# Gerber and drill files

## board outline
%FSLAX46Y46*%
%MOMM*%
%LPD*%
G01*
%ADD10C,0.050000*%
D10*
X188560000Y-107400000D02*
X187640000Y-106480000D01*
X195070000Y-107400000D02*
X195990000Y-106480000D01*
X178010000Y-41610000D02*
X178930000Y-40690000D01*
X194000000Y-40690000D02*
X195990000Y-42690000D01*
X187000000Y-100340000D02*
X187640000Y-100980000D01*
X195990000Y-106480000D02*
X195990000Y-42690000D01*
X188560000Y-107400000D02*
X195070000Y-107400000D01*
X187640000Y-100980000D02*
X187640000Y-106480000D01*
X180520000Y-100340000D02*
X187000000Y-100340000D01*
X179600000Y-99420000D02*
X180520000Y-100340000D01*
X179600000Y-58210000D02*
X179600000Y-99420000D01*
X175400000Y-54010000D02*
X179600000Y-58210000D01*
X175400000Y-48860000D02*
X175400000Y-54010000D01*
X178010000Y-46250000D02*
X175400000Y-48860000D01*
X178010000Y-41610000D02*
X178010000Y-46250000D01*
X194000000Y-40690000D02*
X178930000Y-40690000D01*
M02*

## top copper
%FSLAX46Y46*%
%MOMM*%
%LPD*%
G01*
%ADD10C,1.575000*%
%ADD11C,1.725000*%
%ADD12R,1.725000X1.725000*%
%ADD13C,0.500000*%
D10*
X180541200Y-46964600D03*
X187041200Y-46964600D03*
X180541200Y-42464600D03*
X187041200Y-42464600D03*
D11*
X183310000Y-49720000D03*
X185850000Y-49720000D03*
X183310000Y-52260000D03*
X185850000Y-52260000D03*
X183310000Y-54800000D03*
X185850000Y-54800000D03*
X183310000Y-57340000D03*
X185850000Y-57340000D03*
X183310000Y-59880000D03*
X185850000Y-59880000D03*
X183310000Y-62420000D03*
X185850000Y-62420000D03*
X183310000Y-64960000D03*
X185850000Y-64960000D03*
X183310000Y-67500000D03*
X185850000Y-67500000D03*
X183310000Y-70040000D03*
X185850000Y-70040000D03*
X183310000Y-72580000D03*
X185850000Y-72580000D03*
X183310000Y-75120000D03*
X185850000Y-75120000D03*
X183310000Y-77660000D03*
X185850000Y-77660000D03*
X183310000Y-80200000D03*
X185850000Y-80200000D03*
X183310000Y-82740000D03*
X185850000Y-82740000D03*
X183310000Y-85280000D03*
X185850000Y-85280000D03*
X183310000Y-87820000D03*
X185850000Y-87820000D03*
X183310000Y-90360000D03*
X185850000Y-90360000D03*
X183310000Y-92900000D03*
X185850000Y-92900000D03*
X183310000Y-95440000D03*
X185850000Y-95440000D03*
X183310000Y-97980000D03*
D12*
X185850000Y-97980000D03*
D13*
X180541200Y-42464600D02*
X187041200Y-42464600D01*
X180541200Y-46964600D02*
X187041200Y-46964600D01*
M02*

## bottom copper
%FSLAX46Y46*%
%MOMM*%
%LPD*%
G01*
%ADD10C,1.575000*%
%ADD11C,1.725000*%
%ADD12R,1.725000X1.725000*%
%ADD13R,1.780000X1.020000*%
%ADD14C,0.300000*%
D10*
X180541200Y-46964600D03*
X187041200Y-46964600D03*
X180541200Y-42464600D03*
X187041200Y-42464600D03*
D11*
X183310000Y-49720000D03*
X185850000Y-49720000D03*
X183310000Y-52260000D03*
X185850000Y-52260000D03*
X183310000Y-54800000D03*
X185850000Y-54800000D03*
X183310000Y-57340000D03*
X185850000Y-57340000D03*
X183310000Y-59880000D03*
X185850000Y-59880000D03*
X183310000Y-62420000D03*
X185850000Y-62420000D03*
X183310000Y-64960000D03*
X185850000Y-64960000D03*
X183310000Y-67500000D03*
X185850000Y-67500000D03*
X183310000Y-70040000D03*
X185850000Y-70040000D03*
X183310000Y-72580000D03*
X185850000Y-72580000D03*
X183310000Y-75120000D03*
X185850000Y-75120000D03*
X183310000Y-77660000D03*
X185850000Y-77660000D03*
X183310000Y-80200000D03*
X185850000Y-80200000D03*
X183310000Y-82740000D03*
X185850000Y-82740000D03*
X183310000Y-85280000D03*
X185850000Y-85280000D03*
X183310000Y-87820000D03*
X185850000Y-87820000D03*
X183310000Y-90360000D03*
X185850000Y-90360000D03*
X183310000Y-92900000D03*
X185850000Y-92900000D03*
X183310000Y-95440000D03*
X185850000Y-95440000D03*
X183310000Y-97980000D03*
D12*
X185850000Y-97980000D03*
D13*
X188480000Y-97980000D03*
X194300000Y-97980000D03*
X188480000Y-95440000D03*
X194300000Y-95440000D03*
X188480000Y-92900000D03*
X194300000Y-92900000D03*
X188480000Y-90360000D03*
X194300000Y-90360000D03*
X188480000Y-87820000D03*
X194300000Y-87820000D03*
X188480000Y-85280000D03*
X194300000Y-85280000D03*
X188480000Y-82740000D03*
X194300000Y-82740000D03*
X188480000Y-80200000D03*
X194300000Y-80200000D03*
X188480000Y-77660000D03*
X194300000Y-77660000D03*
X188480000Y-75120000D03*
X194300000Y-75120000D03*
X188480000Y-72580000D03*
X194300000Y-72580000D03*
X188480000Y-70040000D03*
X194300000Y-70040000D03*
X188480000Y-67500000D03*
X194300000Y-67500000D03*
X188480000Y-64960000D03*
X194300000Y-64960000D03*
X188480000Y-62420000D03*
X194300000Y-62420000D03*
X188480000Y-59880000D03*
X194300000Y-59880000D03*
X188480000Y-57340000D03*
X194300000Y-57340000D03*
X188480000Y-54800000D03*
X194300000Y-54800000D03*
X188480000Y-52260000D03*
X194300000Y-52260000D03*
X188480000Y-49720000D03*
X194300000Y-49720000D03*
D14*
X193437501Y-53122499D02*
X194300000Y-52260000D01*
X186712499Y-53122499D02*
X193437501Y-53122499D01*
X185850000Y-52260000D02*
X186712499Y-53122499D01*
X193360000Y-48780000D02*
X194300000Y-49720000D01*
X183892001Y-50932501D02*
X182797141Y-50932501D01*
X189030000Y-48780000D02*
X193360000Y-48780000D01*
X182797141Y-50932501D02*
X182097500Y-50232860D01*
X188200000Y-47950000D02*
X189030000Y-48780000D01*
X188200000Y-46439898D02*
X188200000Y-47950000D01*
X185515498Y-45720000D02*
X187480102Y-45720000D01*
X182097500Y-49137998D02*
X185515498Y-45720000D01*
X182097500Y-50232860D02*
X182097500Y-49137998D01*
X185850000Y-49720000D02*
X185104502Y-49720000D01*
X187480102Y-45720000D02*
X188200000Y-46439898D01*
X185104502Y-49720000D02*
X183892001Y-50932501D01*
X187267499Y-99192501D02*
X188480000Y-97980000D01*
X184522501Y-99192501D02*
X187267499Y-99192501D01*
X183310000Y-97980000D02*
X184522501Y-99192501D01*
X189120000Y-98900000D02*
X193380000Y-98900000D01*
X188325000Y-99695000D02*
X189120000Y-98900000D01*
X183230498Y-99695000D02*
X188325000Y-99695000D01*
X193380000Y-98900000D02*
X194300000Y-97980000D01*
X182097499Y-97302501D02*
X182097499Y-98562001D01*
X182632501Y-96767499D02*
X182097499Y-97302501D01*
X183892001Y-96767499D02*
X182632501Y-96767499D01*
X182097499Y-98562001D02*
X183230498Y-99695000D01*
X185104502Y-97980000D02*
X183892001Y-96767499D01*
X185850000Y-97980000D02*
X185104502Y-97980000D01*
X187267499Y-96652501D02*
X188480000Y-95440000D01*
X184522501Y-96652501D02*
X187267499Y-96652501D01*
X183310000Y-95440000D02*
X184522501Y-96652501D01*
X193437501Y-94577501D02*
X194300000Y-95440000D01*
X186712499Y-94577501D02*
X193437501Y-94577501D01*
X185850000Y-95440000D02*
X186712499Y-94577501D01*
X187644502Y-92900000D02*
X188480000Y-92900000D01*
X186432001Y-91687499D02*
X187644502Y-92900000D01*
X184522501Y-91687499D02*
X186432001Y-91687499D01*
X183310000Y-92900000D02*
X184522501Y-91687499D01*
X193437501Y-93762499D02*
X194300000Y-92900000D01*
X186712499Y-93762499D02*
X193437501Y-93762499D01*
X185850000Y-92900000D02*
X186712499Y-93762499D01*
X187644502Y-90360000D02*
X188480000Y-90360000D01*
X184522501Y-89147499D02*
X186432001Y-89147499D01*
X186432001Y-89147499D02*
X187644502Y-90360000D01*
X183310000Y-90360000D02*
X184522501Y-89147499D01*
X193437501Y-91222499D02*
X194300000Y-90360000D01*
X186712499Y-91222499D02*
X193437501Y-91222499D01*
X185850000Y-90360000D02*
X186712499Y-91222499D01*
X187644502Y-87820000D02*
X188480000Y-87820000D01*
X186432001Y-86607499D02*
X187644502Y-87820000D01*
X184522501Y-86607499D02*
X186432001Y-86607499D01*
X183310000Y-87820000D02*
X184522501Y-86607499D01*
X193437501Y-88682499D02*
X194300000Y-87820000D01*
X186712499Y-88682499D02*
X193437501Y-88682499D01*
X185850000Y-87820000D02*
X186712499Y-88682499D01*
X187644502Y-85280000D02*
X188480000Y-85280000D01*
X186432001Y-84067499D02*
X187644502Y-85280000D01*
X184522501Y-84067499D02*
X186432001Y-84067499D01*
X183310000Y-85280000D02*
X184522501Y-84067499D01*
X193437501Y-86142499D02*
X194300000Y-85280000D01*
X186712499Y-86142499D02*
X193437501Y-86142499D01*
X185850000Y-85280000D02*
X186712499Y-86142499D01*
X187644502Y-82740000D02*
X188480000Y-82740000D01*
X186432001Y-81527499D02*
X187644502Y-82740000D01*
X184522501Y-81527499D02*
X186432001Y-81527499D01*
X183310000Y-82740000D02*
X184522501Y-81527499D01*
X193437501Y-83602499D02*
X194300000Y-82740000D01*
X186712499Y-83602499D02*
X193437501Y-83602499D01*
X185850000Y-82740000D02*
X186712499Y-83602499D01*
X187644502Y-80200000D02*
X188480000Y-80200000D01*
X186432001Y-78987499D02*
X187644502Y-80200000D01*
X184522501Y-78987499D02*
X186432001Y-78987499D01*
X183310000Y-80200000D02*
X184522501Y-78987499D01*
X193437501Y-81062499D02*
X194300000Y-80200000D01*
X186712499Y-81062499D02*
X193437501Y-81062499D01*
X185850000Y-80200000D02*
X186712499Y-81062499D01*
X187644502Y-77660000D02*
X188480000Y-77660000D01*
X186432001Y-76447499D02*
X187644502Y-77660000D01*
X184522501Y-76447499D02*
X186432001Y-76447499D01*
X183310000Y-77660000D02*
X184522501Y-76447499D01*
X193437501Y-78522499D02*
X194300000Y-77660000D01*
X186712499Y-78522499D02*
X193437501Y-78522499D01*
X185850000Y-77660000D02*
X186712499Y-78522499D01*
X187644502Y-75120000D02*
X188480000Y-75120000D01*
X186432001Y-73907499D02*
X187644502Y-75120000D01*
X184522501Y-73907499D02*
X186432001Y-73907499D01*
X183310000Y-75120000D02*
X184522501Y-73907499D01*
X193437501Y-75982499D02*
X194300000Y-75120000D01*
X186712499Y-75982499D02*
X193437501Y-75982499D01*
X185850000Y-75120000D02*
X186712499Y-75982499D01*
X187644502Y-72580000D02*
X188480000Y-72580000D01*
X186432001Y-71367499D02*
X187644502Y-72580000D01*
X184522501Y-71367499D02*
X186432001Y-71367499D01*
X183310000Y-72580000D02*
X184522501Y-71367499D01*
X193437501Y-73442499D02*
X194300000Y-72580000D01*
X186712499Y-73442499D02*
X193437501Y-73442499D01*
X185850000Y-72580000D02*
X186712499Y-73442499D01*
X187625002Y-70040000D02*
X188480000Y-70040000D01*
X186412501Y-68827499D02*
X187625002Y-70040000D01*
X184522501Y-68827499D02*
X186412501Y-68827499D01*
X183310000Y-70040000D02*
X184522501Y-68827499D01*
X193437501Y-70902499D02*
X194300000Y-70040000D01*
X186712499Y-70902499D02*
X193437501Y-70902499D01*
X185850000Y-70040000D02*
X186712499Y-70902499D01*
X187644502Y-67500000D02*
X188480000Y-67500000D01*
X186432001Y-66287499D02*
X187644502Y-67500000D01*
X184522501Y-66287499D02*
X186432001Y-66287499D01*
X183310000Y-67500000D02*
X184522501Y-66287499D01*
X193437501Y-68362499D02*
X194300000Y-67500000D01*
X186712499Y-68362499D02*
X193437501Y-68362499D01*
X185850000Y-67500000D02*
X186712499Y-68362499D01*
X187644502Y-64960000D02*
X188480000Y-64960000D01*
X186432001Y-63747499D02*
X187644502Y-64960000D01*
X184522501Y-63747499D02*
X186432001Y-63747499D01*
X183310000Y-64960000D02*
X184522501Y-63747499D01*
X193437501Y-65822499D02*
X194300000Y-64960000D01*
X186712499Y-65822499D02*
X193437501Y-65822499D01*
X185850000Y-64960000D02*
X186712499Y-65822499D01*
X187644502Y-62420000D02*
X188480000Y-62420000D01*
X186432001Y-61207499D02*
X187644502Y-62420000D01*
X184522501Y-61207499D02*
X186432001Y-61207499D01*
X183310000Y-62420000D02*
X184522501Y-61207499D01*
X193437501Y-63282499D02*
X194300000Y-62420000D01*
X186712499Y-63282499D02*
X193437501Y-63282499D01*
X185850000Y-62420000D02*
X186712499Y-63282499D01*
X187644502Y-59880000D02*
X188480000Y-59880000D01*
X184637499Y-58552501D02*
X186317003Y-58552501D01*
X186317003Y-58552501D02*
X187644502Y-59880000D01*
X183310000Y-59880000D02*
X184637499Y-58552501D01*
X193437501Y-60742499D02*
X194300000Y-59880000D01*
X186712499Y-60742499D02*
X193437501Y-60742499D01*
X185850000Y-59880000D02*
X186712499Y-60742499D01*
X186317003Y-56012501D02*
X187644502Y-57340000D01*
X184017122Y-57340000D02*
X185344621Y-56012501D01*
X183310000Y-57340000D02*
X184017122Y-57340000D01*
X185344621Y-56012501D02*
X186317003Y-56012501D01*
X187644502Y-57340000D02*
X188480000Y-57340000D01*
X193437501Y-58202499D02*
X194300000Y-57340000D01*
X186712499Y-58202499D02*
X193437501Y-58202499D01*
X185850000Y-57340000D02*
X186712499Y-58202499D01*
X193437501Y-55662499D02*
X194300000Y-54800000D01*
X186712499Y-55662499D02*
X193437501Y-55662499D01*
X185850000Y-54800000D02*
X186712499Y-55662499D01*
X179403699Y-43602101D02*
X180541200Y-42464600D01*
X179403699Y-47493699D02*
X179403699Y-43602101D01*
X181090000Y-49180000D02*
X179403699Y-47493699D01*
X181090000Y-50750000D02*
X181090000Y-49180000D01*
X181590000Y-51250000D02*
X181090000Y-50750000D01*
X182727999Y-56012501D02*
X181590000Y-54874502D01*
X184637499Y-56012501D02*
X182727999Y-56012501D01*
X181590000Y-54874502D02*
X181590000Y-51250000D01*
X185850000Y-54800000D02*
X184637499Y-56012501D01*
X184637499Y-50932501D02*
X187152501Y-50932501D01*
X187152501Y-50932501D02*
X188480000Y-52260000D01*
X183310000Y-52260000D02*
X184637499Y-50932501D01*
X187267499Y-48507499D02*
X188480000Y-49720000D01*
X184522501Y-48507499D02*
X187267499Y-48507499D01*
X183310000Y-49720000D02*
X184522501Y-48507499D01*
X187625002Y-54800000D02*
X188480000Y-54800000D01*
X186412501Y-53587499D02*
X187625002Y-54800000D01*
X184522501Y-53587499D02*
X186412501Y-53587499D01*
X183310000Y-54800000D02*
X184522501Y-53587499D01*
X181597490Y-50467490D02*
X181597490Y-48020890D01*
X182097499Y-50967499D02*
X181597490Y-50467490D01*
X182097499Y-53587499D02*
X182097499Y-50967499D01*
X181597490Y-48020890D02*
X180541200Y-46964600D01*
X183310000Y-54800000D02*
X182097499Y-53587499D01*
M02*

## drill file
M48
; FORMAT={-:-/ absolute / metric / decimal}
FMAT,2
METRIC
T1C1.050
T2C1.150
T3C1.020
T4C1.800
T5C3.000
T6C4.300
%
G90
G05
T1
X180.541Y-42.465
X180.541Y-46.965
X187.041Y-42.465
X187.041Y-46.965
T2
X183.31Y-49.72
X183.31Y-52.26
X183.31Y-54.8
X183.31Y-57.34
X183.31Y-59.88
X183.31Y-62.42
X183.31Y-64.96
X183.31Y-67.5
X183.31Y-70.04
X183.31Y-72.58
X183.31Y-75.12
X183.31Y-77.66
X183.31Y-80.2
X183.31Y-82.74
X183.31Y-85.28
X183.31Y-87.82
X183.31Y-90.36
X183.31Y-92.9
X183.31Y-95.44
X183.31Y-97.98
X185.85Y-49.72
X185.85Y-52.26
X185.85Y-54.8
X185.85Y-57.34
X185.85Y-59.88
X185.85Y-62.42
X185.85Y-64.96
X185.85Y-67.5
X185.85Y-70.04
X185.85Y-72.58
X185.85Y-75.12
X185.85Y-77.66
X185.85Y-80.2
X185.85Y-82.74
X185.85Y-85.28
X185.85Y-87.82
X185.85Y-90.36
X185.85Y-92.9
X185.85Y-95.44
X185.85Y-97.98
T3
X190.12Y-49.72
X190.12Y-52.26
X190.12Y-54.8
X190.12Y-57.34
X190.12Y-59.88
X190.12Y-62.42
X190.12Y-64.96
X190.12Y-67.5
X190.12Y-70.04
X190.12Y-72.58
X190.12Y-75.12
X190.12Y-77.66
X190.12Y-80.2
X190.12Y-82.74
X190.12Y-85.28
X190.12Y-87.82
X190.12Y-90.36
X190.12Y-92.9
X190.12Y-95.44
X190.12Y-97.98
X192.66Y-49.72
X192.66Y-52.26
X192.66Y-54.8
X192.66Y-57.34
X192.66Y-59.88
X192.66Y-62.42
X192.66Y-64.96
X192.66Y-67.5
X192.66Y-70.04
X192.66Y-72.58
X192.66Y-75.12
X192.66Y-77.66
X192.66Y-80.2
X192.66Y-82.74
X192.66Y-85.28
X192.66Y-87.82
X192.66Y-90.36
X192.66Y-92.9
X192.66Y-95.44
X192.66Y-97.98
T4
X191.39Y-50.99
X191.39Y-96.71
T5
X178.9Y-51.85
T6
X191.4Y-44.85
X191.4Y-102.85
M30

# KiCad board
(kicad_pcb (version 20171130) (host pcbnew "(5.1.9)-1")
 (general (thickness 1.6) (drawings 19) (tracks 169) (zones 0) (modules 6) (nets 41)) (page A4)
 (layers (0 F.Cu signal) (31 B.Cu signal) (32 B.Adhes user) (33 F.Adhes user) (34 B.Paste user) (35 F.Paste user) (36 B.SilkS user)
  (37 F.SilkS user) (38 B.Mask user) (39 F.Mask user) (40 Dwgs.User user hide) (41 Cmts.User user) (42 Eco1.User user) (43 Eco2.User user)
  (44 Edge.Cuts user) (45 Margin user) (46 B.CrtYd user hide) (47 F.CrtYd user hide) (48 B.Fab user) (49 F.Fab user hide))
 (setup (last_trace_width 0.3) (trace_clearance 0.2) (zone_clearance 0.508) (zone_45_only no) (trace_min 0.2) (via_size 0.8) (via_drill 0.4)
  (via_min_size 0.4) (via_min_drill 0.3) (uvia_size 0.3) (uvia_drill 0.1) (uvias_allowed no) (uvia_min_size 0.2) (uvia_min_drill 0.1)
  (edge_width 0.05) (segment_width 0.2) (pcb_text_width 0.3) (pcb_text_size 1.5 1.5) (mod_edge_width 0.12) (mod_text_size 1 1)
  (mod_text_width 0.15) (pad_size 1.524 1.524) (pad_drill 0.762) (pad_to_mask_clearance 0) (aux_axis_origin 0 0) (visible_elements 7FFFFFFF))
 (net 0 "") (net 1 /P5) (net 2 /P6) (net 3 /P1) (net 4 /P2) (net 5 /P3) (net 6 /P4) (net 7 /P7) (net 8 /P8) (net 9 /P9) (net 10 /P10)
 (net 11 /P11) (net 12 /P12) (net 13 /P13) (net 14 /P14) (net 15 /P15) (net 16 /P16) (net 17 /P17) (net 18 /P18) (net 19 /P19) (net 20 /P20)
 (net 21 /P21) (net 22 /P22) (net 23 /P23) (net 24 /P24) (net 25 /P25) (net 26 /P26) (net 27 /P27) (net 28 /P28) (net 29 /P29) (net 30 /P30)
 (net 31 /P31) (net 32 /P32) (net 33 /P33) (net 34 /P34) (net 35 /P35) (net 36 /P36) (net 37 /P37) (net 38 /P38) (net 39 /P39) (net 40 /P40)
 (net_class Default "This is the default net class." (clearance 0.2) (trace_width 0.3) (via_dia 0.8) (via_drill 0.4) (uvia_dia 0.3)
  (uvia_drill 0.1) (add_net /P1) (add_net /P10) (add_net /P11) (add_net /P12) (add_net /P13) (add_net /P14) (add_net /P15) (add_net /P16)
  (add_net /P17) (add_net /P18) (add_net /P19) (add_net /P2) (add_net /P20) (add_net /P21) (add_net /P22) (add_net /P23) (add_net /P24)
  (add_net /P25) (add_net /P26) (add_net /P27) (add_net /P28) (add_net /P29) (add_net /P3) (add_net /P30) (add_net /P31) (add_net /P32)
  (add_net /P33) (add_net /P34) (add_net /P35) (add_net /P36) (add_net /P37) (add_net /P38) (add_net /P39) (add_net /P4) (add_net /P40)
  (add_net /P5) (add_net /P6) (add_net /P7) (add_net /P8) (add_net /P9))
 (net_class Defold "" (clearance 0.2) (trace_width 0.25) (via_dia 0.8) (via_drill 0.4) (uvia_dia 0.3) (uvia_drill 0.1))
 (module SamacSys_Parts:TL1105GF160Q (layer F.Cu) (at 183.7912 44.7146)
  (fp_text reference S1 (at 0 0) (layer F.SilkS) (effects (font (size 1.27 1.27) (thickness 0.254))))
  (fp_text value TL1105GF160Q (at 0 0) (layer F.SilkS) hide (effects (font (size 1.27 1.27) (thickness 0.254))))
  (pad 1 thru_hole circle (at -3.25 2.25) (size 1.575 1.575) (drill 1.05) (layers *.Cu *.Mask) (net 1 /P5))
  (pad 2 thru_hole circle (at 3.25 2.25) (size 1.575 1.575) (drill 1.05) (layers *.Cu *.Mask) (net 1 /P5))
  (pad 3 thru_hole circle (at -3.25 -2.25) (size 1.575 1.575) (drill 1.05) (layers *.Cu *.Mask) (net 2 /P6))
  (pad 4 thru_hole circle (at 3.25 -2.25) (size 1.575 1.575) (drill 1.05) (layers *.Cu *.Mask) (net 2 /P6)))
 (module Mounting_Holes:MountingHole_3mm (layer F.Cu) (at 178.9 51.85)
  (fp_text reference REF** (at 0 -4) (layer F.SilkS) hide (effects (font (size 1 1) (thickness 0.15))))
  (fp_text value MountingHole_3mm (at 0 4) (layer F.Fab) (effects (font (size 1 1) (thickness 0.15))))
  (pad 1 np_thru_hole circle (at 0 0) (size 3 3) (drill 3) (layers *.Cu *.Mask)))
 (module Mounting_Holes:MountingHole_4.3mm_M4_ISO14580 (layer F.Cu) (at 191.4 102.85)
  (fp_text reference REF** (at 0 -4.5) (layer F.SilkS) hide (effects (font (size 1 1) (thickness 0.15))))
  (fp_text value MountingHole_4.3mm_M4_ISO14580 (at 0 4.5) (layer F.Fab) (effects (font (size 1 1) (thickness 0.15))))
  (pad 1 np_thru_hole circle (at 0 0) (size 4.3 4.3) (drill 4.3) (layers *.Cu *.Mask)))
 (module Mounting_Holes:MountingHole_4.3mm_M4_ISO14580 (layer F.Cu) (at 191.4 44.85)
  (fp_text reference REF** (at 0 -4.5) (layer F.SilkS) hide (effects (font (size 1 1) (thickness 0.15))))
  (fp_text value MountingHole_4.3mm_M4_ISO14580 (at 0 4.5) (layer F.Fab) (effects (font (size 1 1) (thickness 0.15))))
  (pad 1 np_thru_hole circle (at 0 0) (size 4.3 4.3) (drill 4.3) (layers *.Cu *.Mask)))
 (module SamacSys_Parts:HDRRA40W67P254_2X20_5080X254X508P (layer F.Cu) (at 185.85 97.98 270)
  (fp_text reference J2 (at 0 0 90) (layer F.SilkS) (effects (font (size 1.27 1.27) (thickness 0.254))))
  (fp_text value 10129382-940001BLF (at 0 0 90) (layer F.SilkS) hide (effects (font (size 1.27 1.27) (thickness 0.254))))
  (pad 40 thru_hole circle (at -48.26 2.54 270) (size 1.725 1.725) (drill 1.15) (layers *.Cu *.Mask) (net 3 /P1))
  (pad 39 thru_hole circle (at -48.26 0 270) (size 1.725 1.725) (drill 1.15) (layers *.Cu *.Mask) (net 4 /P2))
  (pad 38 thru_hole circle (at -45.72 2.54 270) (size 1.725 1.725) (drill 1.15) (layers *.Cu *.Mask) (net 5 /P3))
  (pad 37 thru_hole circle (at -45.72 0 270) (size 1.725 1.725) (drill 1.15) (layers *.Cu *.Mask) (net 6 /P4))
  (pad 36 thru_hole circle (at -43.18 2.54 270) (size 1.725 1.725) (drill 1.15) (layers *.Cu *.Mask) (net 1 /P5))
  (pad 35 thru_hole circle (at -43.18 0 270) (size 1.725 1.725) (drill 1.15) (layers *.Cu *.Mask) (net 2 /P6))
  (pad 34 thru_hole circle (at -40.64 2.54 270) (size 1.725 1.725) (drill 1.15) (layers *.Cu *.Mask) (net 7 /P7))
  (pad 33 thru_hole circle (at -40.64 0 270) (size 1.725 1.725) (drill 1.15) (layers *.Cu *.Mask) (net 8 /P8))
  (pad 32 thru_hole circle (at -38.1 2.54 270) (size 1.725 1.725) (drill 1.15) (layers *.Cu *.Mask) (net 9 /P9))
  (pad 31 thru_hole circle (at -38.1 0 270) (size 1.725 1.725) (drill 1.15) (layers *.Cu *.Mask) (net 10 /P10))
  (pad 30 thru_hole circle (at -35.56 2.54 270) (size 1.725 1.725) (drill 1.15) (layers *.Cu *.Mask) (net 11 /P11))
  (pad 29 thru_hole circle (at -35.56 0 270) (size 1.725 1.725) (drill 1.15) (layers *.Cu *.Mask) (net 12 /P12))
  (pad 28 thru_hole circle (at -33.02 2.54 270) (size 1.725 1.725) (drill 1.15) (layers *.Cu *.Mask) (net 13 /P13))
  (pad 27 thru_hole circle (at -33.02 0 270) (size 1.725 1.725) (drill 1.15) (layers *.Cu *.Mask) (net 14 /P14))
  (pad 26 thru_hole circle (at -30.48 2.54 270) (size 1.725 1.725) (drill 1.15) (layers *.Cu *.Mask) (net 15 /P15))
  (pad 25 thru_hole circle (at -30.48 0 270) (size 1.725 1.725) (drill 1.15) (layers *.Cu *.Mask) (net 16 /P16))
  (pad 24 thru_hole circle (at -27.94 2.54 270) (size 1.725 1.725) (drill 1.15) (layers *.Cu *.Mask) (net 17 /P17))
  (pad 23 thru_hole circle (at -27.94 0 270) (size 1.725 1.725) (drill 1.15) (layers *.Cu *.Mask) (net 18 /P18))
  (pad 22 thru_hole circle (at -25.4 2.54 270) (size 1.725 1.725) (drill 1.15) (layers *.Cu *.Mask) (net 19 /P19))
  (pad 21 thru_hole circle (at -25.4 0 270) (size 1.725 1.725) (drill 1.15) (layers *.Cu *.Mask) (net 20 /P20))
  (pad 20 thru_hole circle (at -22.86 2.54 270) (size 1.725 1.725) (drill 1.15) (layers *.Cu *.Mask) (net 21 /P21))
  (pad 19 thru_hole circle (at -22.86 0 270) (size 1.725 1.725) (drill 1.15) (layers *.Cu *.Mask) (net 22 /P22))
  (pad 18 thru_hole circle (at -20.32 2.54 270) (size 1.725 1.725) (drill 1.15) (layers *.Cu *.Mask) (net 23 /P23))
  (pad 17 thru_hole circle (at -20.32 0 270) (size 1.725 1.725) (drill 1.15) (layers *.Cu *.Mask) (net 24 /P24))
  (pad 16 thru_hole circle (at -17.78 2.54 270) (size 1.725 1.725) (drill 1.15) (layers *.Cu *.Mask) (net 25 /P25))
  (pad 15 thru_hole circle (at -17.78 0 270) (size 1.725 1.725) (drill 1.15) (layers *.Cu *.Mask) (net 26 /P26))
  (pad 14 thru_hole circle (at -15.24 2.54 270) (size 1.725 1.725) (drill 1.15) (layers *.Cu *.Mask) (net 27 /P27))
  (pad 13 thru_hole circle (at -15.24 0 270) (size 1.725 1.725) (drill 1.15) (layers *.Cu *.Mask) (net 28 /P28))
  (pad 12 thru_hole circle (at -12.7 2.54 270) (size 1.725 1.725) (drill 1.15) (layers *.Cu *.Mask) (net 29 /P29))
  (pad 11 thru_hole circle (at -12.7 0 270) (size 1.725 1.725) (drill 1.15) (layers *.Cu *.Mask) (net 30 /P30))
  (pad 10 thru_hole circle (at -10.16 2.54 270) (size 1.725 1.725) (drill 1.15) (layers *.Cu *.Mask) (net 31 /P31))
  (pad 9 thru_hole circle (at -10.16 0 270) (size 1.725 1.725) (drill 1.15) (layers *.Cu *.Mask) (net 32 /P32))
  (pad 8 thru_hole circle (at -7.62 2.54 270) (size 1.725 1.725) (drill 1.15) (layers *.Cu *.Mask) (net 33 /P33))
  (pad 7 thru_hole circle (at -7.62 0 270) (size 1.725 1.725) (drill 1.15) (layers *.Cu *.Mask) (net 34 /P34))
  (pad 6 thru_hole circle (at -5.08 2.54 270) (size 1.725 1.725) (drill 1.15) (layers *.Cu *.Mask) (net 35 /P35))
  (pad 5 thru_hole circle (at -5.08 0 270) (size 1.725 1.725) (drill 1.15) (layers *.Cu *.Mask) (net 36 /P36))
  (pad 4 thru_hole circle (at -2.54 2.54 270) (size 1.725 1.725) (drill 1.15) (layers *.Cu *.Mask) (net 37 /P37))
  (pad 3 thru_hole circle (at -2.54 0 270) (size 1.725 1.725) (drill 1.15) (layers *.Cu *.Mask) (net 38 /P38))
  (pad 2 thru_hole circle (at 0 2.54 270) (size 1.725 1.725) (drill 1.15) (layers *.Cu *.Mask) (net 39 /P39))
  (pad 1 thru_hole rect (at 0 0 270) (size 1.725 1.725) (drill 1.15) (layers *.Cu *.Mask) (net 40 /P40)))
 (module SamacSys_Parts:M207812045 (layer B.Cu) (at 191.39 73.85 270)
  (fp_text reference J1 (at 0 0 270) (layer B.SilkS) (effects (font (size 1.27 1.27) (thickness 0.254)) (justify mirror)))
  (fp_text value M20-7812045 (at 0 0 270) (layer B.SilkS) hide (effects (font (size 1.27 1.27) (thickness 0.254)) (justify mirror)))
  (pad MH2 np_thru_hole circle (at 22.86 0 270) (size 1.8 0) (drill 1.8) (layers *.Cu *.Mask))
  (pad MH1 np_thru_hole circle (at -22.86 0 270) (size 1.8 0) (drill 1.8) (layers *.Cu *.Mask))
  (pad 80 np_thru_hole circle (at 24.13 1.27 270) (size 1.02 0) (drill 1.02) (layers *.Cu *.Mask))
  (pad 79 np_thru_hole circle (at 24.13 -1.27 270) (size 1.02 0) (drill 1.02) (layers *.Cu *.Mask))
  (pad 78 np_thru_hole circle (at 21.59 1.27 270) (size 1.02 0) (drill 1.02) (layers *.Cu *.Mask))
  (pad 77 np_thru_hole circle (at 21.59 -1.27 270) (size 1.02 0) (drill 1.02) (layers *.Cu *.Mask))
  (pad 76 np_thru_hole circle (at 19.05 1.27 270) (size 1.02 0) (drill 1.02) (layers *.Cu *.Mask))
  (pad 75 np_thru_hole circle (at 19.05 -1.27 270) (size 1.02 0) (drill 1.02) (layers *.Cu *.Mask))
  (pad 74 np_thru_hole circle (at 16.51 1.27 270) (size 1.02 0) (drill 1.02) (layers *.Cu *.Mask))
  (pad 73 np_thru_hole circle (at 16.51 -1.27 270) (size 1.02 0) (drill 1.02) (layers *.Cu *.Mask))
  (pad 72 np_thru_hole circle (at 13.97 1.27 270) (size 1.02 0) (drill 1.02) (layers *.Cu *.Mask))
  (pad 71 np_thru_hole circle (at 13.97 -1.27 270) (size 1.02 0) (drill 1.02) (layers *.Cu *.Mask))
  (pad 70 np_thru_hole circle (at 11.43 1.27 270) (size 1.02 0) (drill 1.02) (layers *.Cu *.Mask))
  (pad 69 np_thru_hole circle (at 11.43 -1.27 270) (size 1.02 0) (drill 1.02) (layers *.Cu *.Mask))
  (pad 68 np_thru_hole circle (at 8.89 1.27 270) (size 1.02 0) (drill 1.02) (layers *.Cu *.Mask))
  (pad 67 np_thru_hole circle (at 8.89 -1.27 270) (size 1.02 0) (drill 1.02) (layers *.Cu *.Mask))
  (pad 66 np_thru_hole circle (at 6.35 1.27 270) (size 1.02 0) (drill 1.02) (layers *.Cu *.Mask))
  (pad 65 np_thru_hole circle (at 6.35 -1.27 270) (size 1.02 0) (drill 1.02) (layers *.Cu *.Mask))
  (pad 64 np_thru_hole circle (at 3.81 1.27 270) (size 1.02 0) (drill 1.02) (layers *.Cu *.Mask))
  (pad 63 np_thru_hole circle (at 3.81 -1.27 270) (size 1.02 0) (drill 1.02) (layers *.Cu *.Mask))
  (pad 62 np_thru_hole circle (at 1.27 1.27 270) (size 1.02 0) (drill 1.02) (layers *.Cu *.Mask))
  (pad 61 np_thru_hole circle (at 1.27 -1.27 270) (size 1.02 0) (drill 1.02) (layers *.Cu *.Mask))
  (pad 60 np_thru_hole circle (at -1.27 1.27 270) (size 1.02 0) (drill 1.02) (layers *.Cu *.Mask))
  (pad 59 np_thru_hole circle (at -1.27 -1.27 270) (size 1.02 0) (drill 1.02) (layers *.Cu *.Mask))
  (pad 58 np_thru_hole circle (at -3.81 1.27 270) (size 1.02 0) (drill 1.02) (layers *.Cu *.Mask))
  (pad 57 np_thru_hole circle (at -3.81 -1.27 270) (size 1.02 0) (drill 1.02) (layers *.Cu *.Mask))
  (pad 56 np_thru_hole circle (at -6.35 1.27 270) (size 1.02 0) (drill 1.02) (layers *.Cu *.Mask))
  (pad 55 np_thru_hole circle (at -6.35 -1.27 270) (size 1.02 0) (drill 1.02) (layers *.Cu *.Mask))
  (pad 54 np_thru_hole circle (at -8.89 1.27 270) (size 1.02 0) (drill 1.02) (layers *.Cu *.Mask))
  (pad 53 np_thru_hole circle (at -8.89 -1.27 270) (size 1.02 0) (drill 1.02) (layers *.Cu *.Mask))
  (pad 52 np_thru_hole circle (at -11.43 1.27 270) (size 1.02 0) (drill 1.02) (layers *.Cu *.Mask))
  (pad 51 np_thru_hole circle (at -11.43 -1.27 270) (size 1.02 0) (drill 1.02) (layers *.Cu *.Mask))
  (pad 50 np_thru_hole circle (at -13.97 1.27 270) (size 1.02 0) (drill 1.02) (layers *.Cu *.Mask))
  (pad 49 np_thru_hole circle (at -13.97 -1.27 270) (size 1.02 0) (drill 1.02) (layers *.Cu *.Mask))
  (pad 48 np_thru_hole circle (at -16.51 1.27 270) (size 1.02 0) (drill 1.02) (layers *.Cu *.Mask))
  (pad 47 np_thru_hole circle (at -16.51 -1.27 270) (size 1.02 0) (drill 1.02) (layers *.Cu *.Mask))
  (pad 46 np_thru_hole circle (at -19.05 1.27 270) (size 1.02 0) (drill 1.02) (layers *.Cu *.Mask))
  (pad 45 np_thru_hole circle (at -19.05 -1.27 270) (size 1.02 0) (drill 1.02) (layers *.Cu *.Mask))
  (pad 44 np_thru_hole circle (at -21.59 1.27 270) (size 1.02 0) (drill 1.02) (layers *.Cu *.Mask))
  (pad 43 np_thru_hole circle (at -21.59 -1.27 270) (size 1.02 0) (drill 1.02) (layers *.Cu *.Mask))
  (pad 42 np_thru_hole circle (at -24.13 1.27 270) (size 1.02 0) (drill 1.02) (layers *.Cu *.Mask))
  (pad 41 np_thru_hole circle (at -24.13 -1.27 270) (size 1.02 0) (drill 1.02) (layers *.Cu *.Mask))
  (pad 40 smd rect (at 24.13 2.91 270) (size 1.02 1.78) (layers B.Cu B.Paste B.Mask) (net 39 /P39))
  (pad 39 smd rect (at 24.13 -2.91 270) (size 1.02 1.78) (layers B.Cu B.Paste B.Mask) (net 40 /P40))
  (pad 38 smd rect (at 21.59 2.91 270) (size 1.02 1.78) (layers B.Cu B.Paste B.Mask) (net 37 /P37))
  (pad 37 smd rect (at 21.59 -2.91 270) (size 1.02 1.78) (layers B.Cu B.Paste B.Mask) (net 38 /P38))
  (pad 36 smd rect (at 19.05 2.91 270) (size 1.02 1.78) (layers B.Cu B.Paste B.Mask) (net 35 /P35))
  (pad 35 smd rect (at 19.05 -2.91 270) (size 1.02 1.78) (layers B.Cu B.Paste B.Mask) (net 36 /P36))
  (pad 34 smd rect (at 16.51 2.91 270) (size 1.02 1.78) (layers B.Cu B.Paste B.Mask) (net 33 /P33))
  (pad 33 smd rect (at 16.51 -2.91 270) (size 1.02 1.78) (layers B.Cu B.Paste B.Mask) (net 34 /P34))
  (pad 32 smd rect (at 13.97 2.91 270) (size 1.02 1.78) (layers B.Cu B.Paste B.Mask) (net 31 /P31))
  (pad 31 smd rect (at 13.97 -2.91 270) (size 1.02 1.78) (layers B.Cu B.Paste B.Mask) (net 32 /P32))
  (pad 30 smd rect (at 11.43 2.91 270) (size 1.02 1.78) (layers B.Cu B.Paste B.Mask) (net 29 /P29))
  (pad 29 smd rect (at 11.43 -2.91 270) (size 1.02 1.78) (layers B.Cu B.Paste B.Mask) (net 30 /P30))
  (pad 28 smd rect (at 8.89 2.91 270) (size 1.02 1.78) (layers B.Cu B.Paste B.Mask) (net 27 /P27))
  (pad 27 smd rect (at 8.89 -2.91 270) (size 1.02 1.78) (layers B.Cu B.Paste B.Mask) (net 28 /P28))
  (pad 26 smd rect (at 6.35 2.91 270) (size 1.02 1.78) (layers B.Cu B.Paste B.Mask) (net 25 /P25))
  (pad 25 smd rect (at 6.35 -2.91 270) (size 1.02 1.78) (layers B.Cu B.Paste B.Mask) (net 26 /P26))
  (pad 24 smd rect (at 3.81 2.91 270) (size 1.02 1.78) (layers B.Cu B.Paste B.Mask) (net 23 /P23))
  (pad 23 smd rect (at 3.81 -2.91 270) (size 1.02 1.78) (layers B.Cu B.Paste B.Mask) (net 24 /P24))
  (pad 22 smd rect (at 1.27 2.91 270) (size 1.02 1.78) (layers B.Cu B.Paste B.Mask) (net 21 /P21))
  (pad 21 smd rect (at 1.27 -2.91 270) (size 1.02 1.78) (layers B.Cu B.Paste B.Mask) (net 22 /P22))
  (pad 20 smd rect (at -1.27 2.91 270) (size 1.02 1.78) (layers B.Cu B.Paste B.Mask) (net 19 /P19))
  (pad 19 smd rect (at -1.27 -2.91 270) (size 1.02 1.78) (layers B.Cu B.Paste B.Mask) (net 20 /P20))
  (pad 18 smd rect (at -3.81 2.91 270) (size 1.02 1.78) (layers B.Cu B.Paste B.Mask) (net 17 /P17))
  (pad 17 smd rect (at -3.81 -2.91 270) (size 1.02 1.78) (layers B.Cu B.Paste B.Mask) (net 18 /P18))
  (pad 16 smd rect (at -6.35 2.91 270) (size 1.02 1.78) (layers B.Cu B.Paste B.Mask) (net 15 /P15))
  (pad 15 smd rect (at -6.35 -2.91 270) (size 1.02 1.78) (layers B.Cu B.Paste B.Mask) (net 16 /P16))
  (pad 14 smd rect (at -8.89 2.91 270) (size 1.02 1.78) (layers B.Cu B.Paste B.Mask) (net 13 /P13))
  (pad 13 smd rect (at -8.89 -2.91 270) (size 1.02 1.78) (layers B.Cu B.Paste B.Mask) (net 14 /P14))
  (pad 12 smd rect (at -11.43 2.91 270) (size 1.02 1.78) (layers B.Cu B.Paste B.Mask) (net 11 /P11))
  (pad 11 smd rect (at -11.43 -2.91 270) (size 1.02 1.78) (layers B.Cu B.Paste B.Mask) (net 12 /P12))
  (pad 10 smd rect (at -13.97 2.91 270) (size 1.02 1.78) (layers B.Cu B.Paste B.Mask) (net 9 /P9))
  (pad 9 smd rect (at -13.97 -2.91 270) (size 1.02 1.78) (layers B.Cu B.Paste B.Mask) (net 10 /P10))
  (pad 8 smd rect (at -16.51 2.91 270) (size 1.02 1.78) (layers B.Cu B.Paste B.Mask) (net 7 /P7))
  (pad 7 smd rect (at -16.51 -2.91 270) (size 1.02 1.78) (layers B.Cu B.Paste B.Mask) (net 8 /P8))
  (pad 6 smd rect (at -19.05 2.91 270) (size 1.02 1.78) (layers B.Cu B.Paste B.Mask) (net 1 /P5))
  (pad 5 smd rect (at -19.05 -2.91 270) (size 1.02 1.78) (layers B.Cu B.Paste B.Mask) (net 2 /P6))
  (pad 4 smd rect (at -21.59 2.91 270) (size 1.02 1.78) (layers B.Cu B.Paste B.Mask) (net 5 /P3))
  (pad 3 smd rect (at -21.59 -2.91 270) (size 1.02 1.78) (layers B.Cu B.Paste B.Mask) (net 6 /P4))
  (pad 2 smd rect (at -24.13 2.91 270) (size 1.02 1.78) (layers B.Cu B.Paste B.Mask) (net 3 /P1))
  (pad 1 smd rect (at -24.13 -2.91 270) (size 1.02 1.78) (layers B.Cu B.Paste B.Mask) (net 4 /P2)))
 (gr_line (start 188.56 107.4) (end 187.64 106.48) (layer Edge.Cuts) (width 0.05))
 (gr_line (start 195.07 107.4) (end 195.99 106.48) (layer Edge.Cuts) (width 0.05))
 (gr_line (start 178.01 41.61) (end 178.93 40.69) (layer Edge.Cuts) (width 0.05))
 (gr_line (start 194 40.69) (end 195.99 42.69) (layer Edge.Cuts) (width 0.05))
 (gr_line (start 187 100.34) (end 187.64 100.98) (layer Edge.Cuts) (width 0.05))
 (gr_line (start 195.99 106.48) (end 195.99 42.69) (layer Edge.Cuts) (width 0.05))
 (gr_line (start 188.56 107.4) (end 195.07 107.4) (layer Edge.Cuts) (width 0.05))
 (gr_line (start 187.64 100.98) (end 187.64 106.48) (layer Edge.Cuts) (width 0.05))
 (gr_line (start 180.52 100.34) (end 187 100.34) (layer Edge.Cuts) (width 0.05))
 (gr_line (start 179.6 99.42) (end 180.52 100.34) (layer Edge.Cuts) (width 0.05))
 (gr_line (start 179.6 58.21) (end 179.6 99.42) (layer Edge.Cuts) (width 0.05))
 (gr_line (start 175.4 54.01) (end 179.6 58.21) (layer Edge.Cuts) (width 0.05))
 (gr_line (start 175.4 48.86) (end 175.4 54.01) (layer Edge.Cuts) (width 0.05))
 (gr_line (start 178.01 46.25) (end 175.4 48.86) (layer Edge.Cuts) (width 0.05))
 (gr_line (start 178.01 41.61) (end 178.01 46.25) (layer Edge.Cuts) (width 0.05))
 (gr_line (start 194 40.69) (end 178.93 40.69) (layer Edge.Cuts) (width 0.05))
 (segment (start 193.437501 53.122499) (end 194.3 52.26) (width 0.3) (layer B.Cu) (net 6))
 (segment (start 186.712499 53.122499) (end 193.437501 53.122499) (width 0.3) (layer B.Cu) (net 6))
 (segment (start 185.85 52.26) (end 186.712499 53.122499) (width 0.3) (layer B.Cu) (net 6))
 (segment (start 193.36 48.78) (end 194.3 49.72) (width 0.3) (layer B.Cu) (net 4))
 (segment (start 183.892001 50.932501) (end 182.797141 50.932501) (width 0.3) (layer B.Cu) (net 4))
 (segment (start 189.03 48.78) (end 193.36 48.78) (width 0.3) (layer B.Cu) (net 4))
 (segment (start 182.797141 50.932501) (end 182.0975 50.23286) (width 0.3) (layer B.Cu) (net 4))
 (segment (start 188.2 47.95) (end 189.03 48.78) (width 0.3) (layer B.Cu) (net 4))
 (segment (start 188.2 46.439898) (end 188.2 47.95) (width 0.3) (layer B.Cu) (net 4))
 (segment (start 185.515498 45.72) (end 187.480102 45.72) (width 0.3) (layer B.Cu) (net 4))
 (segment (start 182.0975 49.137998) (end 185.515498 45.72) (width 0.3) (layer B.Cu) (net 4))
 (segment (start 182.0975 50.23286) (end 182.0975 49.137998) (width 0.3) (layer B.Cu) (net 4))
 (segment (start 185.85 49.72) (end 185.104502 49.72) (width 0.3) (layer B.Cu) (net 4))
 (segment (start 187.480102 45.72) (end 188.2 46.439898) (width 0.3) (layer B.Cu) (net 4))
 (segment (start 185.104502 49.72) (end 183.892001 50.932501) (width 0.3) (layer B.Cu) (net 4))
 (segment (start 187.267499 99.192501) (end 188.48 97.98) (width 0.3) (layer B.Cu) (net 39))
 (segment (start 184.522501 99.192501) (end 187.267499 99.192501) (width 0.3) (layer B.Cu) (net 39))
 (segment (start 183.31 97.98) (end 184.522501 99.192501) (width 0.3) (layer B.Cu) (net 39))
 (segment (start 189.12 98.9) (end 193.38 98.9) (width 0.3) (layer B.Cu) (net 40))
 (segment (start 188.325 99.695) (end 189.12 98.9) (width 0.3) (layer B.Cu) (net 40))
 (segment (start 183.230498 99.695) (end 188.325 99.695) (width 0.3) (layer B.Cu) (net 40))
 (segment (start 193.38 98.9) (end 194.3 97.98) (width 0.3) (layer B.Cu) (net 40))
 (segment (start 182.097499 97.302501) (end 182.097499 98.562001) (width 0.3) (layer B.Cu) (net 40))
 (segment (start 182.632501 96.767499) (end 182.097499 97.302501) (width 0.3) (layer B.Cu) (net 40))
 (segment (start 183.892001 96.767499) (end 182.632501 96.767499) (width 0.3) (layer B.Cu) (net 40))
 (segment (start 182.097499 98.562001) (end 183.230498 99.695) (width 0.3) (layer B.Cu) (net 40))
 (segment (start 185.104502 97.98) (end 183.892001 96.767499) (width 0.3) (layer B.Cu) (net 40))
 (segment (start 185.85 97.98) (end 185.104502 97.98) (width 0.3) (layer B.Cu) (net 40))
 (segment (start 187.267499 96.652501) (end 188.48 95.44) (width 0.3) (layer B.Cu) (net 37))
 (segment (start 184.522501 96.652501) (end 187.267499 96.652501) (width 0.3) (layer B.Cu) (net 37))
 (segment (start 183.31 95.44) (end 184.522501 96.652501) (width 0.3) (layer B.Cu) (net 37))
 (segment (start 193.437501 94.577501) (end 194.3 95.44) (width 0.3) (layer B.Cu) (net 38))
 (segment (start 186.712499 94.577501) (end 193.437501 94.577501) (width 0.3) (layer B.Cu) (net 38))
 (segment (start 185.85 95.44) (end 186.712499 94.577501) (width 0.3) (layer B.Cu) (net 38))
 (segment (start 187.644502 92.9) (end 188.48 92.9) (width 0.3) (layer B.Cu) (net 35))
 (segment (start 186.432001 91.687499) (end 187.644502 92.9) (width 0.3) (layer B.Cu) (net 35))
 (segment (start 184.522501 91.687499) (end 186.432001 91.687499) (width 0.3) (layer B.Cu) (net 35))
 (segment (start 183.31 92.9) (end 184.522501 91.687499) (width 0.3) (layer B.Cu) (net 35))
 (segment (start 193.437501 93.762499) (end 194.3 92.9) (width 0.3) (layer B.Cu) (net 36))
 (segment (start 186.712499 93.762499) (end 193.437501 93.762499) (width 0.3) (layer B.Cu) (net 36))
 (segment (start 185.85 92.9) (end 186.712499 93.762499) (width 0.3) (layer B.Cu) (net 36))
 (segment (start 187.644502 90.36) (end 188.48 90.36) (width 0.3) (layer B.Cu) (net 33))
 (segment (start 184.522501 89.147499) (end 186.432001 89.147499) (width 0.3) (layer B.Cu) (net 33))
 (segment (start 186.432001 89.147499) (end 187.644502 90.36) (width 0.3) (layer B.Cu) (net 33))
 (segment (start 183.31 90.36) (end 184.522501 89.147499) (width 0.3) (layer B.Cu) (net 33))
 (segment (start 193.437501 91.222499) (end 194.3 90.36) (width 0.3) (layer B.Cu) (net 34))
 (segment (start 186.712499 91.222499) (end 193.437501 91.222499) (width 0.3) (layer B.Cu) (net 34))
 (segment (start 185.85 90.36) (end 186.712499 91.222499) (width 0.3) (layer B.Cu) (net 34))
 (segment (start 187.644502 87.82) (end 188.48 87.82) (width 0.3) (layer B.Cu) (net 31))
 (segment (start 186.432001 86.607499) (end 187.644502 87.82) (width 0.3) (layer B.Cu) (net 31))
 (segment (start 184.522501 86.607499) (end 186.432001 86.607499) (width 0.3) (layer B.Cu) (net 31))
 (segment (start 183.31 87.82) (end 184.522501 86.607499) (width 0.3) (layer B.Cu) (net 31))
 (segment (start 193.437501 88.682499) (end 194.3 87.82) (width 0.3) (layer B.Cu) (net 32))
 (segment (start 186.712499 88.682499) (end 193.437501 88.682499) (width 0.3) (layer B.Cu) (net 32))
 (segment (start 185.85 87.82) (end 186.712499 88.682499) (width 0.3) (layer B.Cu) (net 32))
 (segment (start 187.644502 85.28) (end 188.48 85.28) (width 0.3) (layer B.Cu) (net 29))
 (segment (start 186.432001 84.067499) (end 187.644502 85.28) (width 0.3) (layer B.Cu) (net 29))
 (segment (start 184.522501 84.067499) (end 186.432001 84.067499) (width 0.3) (layer B.Cu) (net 29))
 (segment (start 183.31 85.28) (end 184.522501 84.067499) (width 0.3) (layer B.Cu) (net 29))
 (segment (start 193.437501 86.142499) (end 194.3 85.28) (width 0.3) (layer B.Cu) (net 30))
 (segment (start 186.712499 86.142499) (end 193.437501 86.142499) (width 0.3) (layer B.Cu) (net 30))
 (segment (start 185.85 85.28) (end 186.712499 86.142499) (width 0.3) (layer B.Cu) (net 30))
 (segment (start 187.644502 82.74) (end 188.48 82.74) (width 0.3) (layer B.Cu) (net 27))
 (segment (start 186.432001 81.527499) (end 187.644502 82.74) (width 0.3) (layer B.Cu) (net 27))
 (segment (start 184.522501 81.527499) (end 186.432001 81.527499) (width 0.3) (layer B.Cu) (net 27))
 (segment (start 183.31 82.74) (end 184.522501 81.527499) (width 0.3) (layer B.Cu) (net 27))
 (segment (start 193.437501 83.602499) (end 194.3 82.74) (width 0.3) (layer B.Cu) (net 28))
 (segment (start 186.712499 83.602499) (end 193.437501 83.602499) (width 0.3) (layer B.Cu) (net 28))
 (segment (start 185.85 82.74) (end 186.712499 83.602499) (width 0.3) (layer B.Cu) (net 28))
 (segment (start 187.644502 80.2) (end 188.48 80.2) (width 0.3) (layer B.Cu) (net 25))
 (segment (start 186.432001 78.987499) (end 187.644502 80.2) (width 0.3) (layer B.Cu) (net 25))
 (segment (start 184.522501 78.987499) (end 186.432001 78.987499) (width 0.3) (layer B.Cu) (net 25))
 (segment (start 183.31 80.2) (end 184.522501 78.987499) (width 0.3) (layer B.Cu) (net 25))
 (segment (start 193.437501 81.062499) (end 194.3 80.2) (width 0.3) (layer B.Cu) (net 26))
 (segment (start 186.712499 81.062499) (end 193.437501 81.062499) (width 0.3) (layer B.Cu) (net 26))
 (segment (start 185.85 80.2) (end 186.712499 81.062499) (width 0.3) (layer B.Cu) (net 26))
 (segment (start 187.644502 77.66) (end 188.48 77.66) (width 0.3) (layer B.Cu) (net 23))
 (segment (start 186.432001 76.447499) (end 187.644502 77.66) (width 0.3) (layer B.Cu) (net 23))
 (segment (start 184.522501 76.447499) (end 186.432001 76.447499) (width 0.3) (layer B.Cu) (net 23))
 (segment (start 183.31 77.66) (end 184.522501 76.447499) (width 0.3) (layer B.Cu) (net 23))
 (segment (start 193.437501 78.522499) (end 194.3 77.66) (width 0.3) (layer B.Cu) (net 24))
 (segment (start 186.712499 78.522499) (end 193.437501 78.522499) (width 0.3) (layer B.Cu) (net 24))
 (segment (start 185.85 77.66) (end 186.712499 78.522499) (width 0.3) (layer B.Cu) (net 24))
 (segment (start 187.644502 75.12) (end 188.48 75.12) (width 0.3) (layer B.Cu) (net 21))
 (segment (start 186.432001 73.907499) (end 187.644502 75.12) (width 0.3) (layer B.Cu) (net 21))
 (segment (start 184.522501 73.907499) (end 186.432001 73.907499) (width 0.3) (layer B.Cu) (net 21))
 (segment (start 183.31 75.12) (end 184.522501 73.907499) (width 0.3) (layer B.Cu) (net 21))
 (segment (start 193.437501 75.982499) (end 194.3 75.12) (width 0.3) (layer B.Cu) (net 22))
 (segment (start 186.712499 75.982499) (end 193.437501 75.982499) (width 0.3) (layer B.Cu) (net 22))
 (segment (start 185.85 75.12) (end 186.712499 75.982499) (width 0.3) (layer B.Cu) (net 22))
 (segment (start 187.644502 72.58) (end 188.48 72.58) (width 0.3) (layer B.Cu) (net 19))
 (segment (start 186.432001 71.367499) (end 187.644502 72.58) (width 0.3) (layer B.Cu) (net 19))
 (segment (start 184.522501 71.367499) (end 186.432001 71.367499) (width 0.3) (layer B.Cu) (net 19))
 (segment (start 183.31 72.58) (end 184.522501 71.367499) (width 0.3) (layer B.Cu) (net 19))
 (segment (start 193.437501 73.442499) (end 194.3 72.58) (width 0.3) (layer B.Cu) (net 20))
 (segment (start 186.712499 73.442499) (end 193.437501 73.442499) (width 0.3) (layer B.Cu) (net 20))
 (segment (start 185.85 72.58) (end 186.712499 73.442499) (width 0.3) (layer B.Cu) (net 20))
 (segment (start 187.625002 70.04) (end 188.48 70.04) (width 0.3) (layer B.Cu) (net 17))
 (segment (start 186.412501 68.827499) (end 187.625002 70.04) (width 0.3) (layer B.Cu) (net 17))
 (segment (start 184.522501 68.827499) (end 186.412501 68.827499) (width 0.3) (layer B.Cu) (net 17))
 (segment (start 183.31 70.04) (end 184.522501 68.827499) (width 0.3) (layer B.Cu) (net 17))
 (segment (start 193.437501 70.902499) (end 194.3 70.04) (width 0.3) (layer B.Cu) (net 18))
 (segment (start 186.712499 70.902499) (end 193.437501 70.902499) (width 0.3) (layer B.Cu) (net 18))
 (segment (start 185.85 70.04) (end 186.712499 70.902499) (width 0.3) (layer B.Cu) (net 18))
 (segment (start 187.644502 67.5) (end 188.48 67.5) (width 0.3) (layer B.Cu) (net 15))
 (segment (start 186.432001 66.287499) (end 187.644502 67.5) (width 0.3) (layer B.Cu) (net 15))
 (segment (start 184.522501 66.287499) (end 186.432001 66.287499) (width 0.3) (layer B.Cu) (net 15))
 (segment (start 183.31 67.5) (end 184.522501 66.287499) (width 0.3) (layer B.Cu) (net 15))
 (segment (start 193.437501 68.362499) (end 194.3 67.5) (width 0.3) (layer B.Cu) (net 16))
 (segment (start 186.712499 68.362499) (end 193.437501 68.362499) (width 0.3) (layer B.Cu) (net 16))
 (segment (start 185.85 67.5) (end 186.712499 68.362499) (width 0.3) (layer B.Cu) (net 16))
 (segment (start 187.644502 64.96) (end 188.48 64.96) (width 0.3) (layer B.Cu) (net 13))
 (segment (start 186.432001 63.747499) (end 187.644502 64.96) (width 0.3) (layer B.Cu) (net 13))
 (segment (start 184.522501 63.747499) (end 186.432001 63.747499) (width 0.3) (layer B.Cu) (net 13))
 (segment (start 183.31 64.96) (end 184.522501 63.747499) (width 0.3) (layer B.Cu) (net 13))
 (segment (start 193.437501 65.822499) (end 194.3 64.96) (width 0.3) (layer B.Cu) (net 14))
 (segment (start 186.712499 65.822499) (end 193.437501 65.822499) (width 0.3) (layer B.Cu) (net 14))
 (segment (start 185.85 64.96) (end 186.712499 65.822499) (width 0.3) (layer B.Cu) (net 14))
 (segment (start 187.644502 62.42) (end 188.48 62.42) (width 0.3) (layer B.Cu) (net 11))
 (segment (start 186.432001 61.207499) (end 187.644502 62.42) (width 0.3) (layer B.Cu) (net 11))
 (segment (start 184.522501 61.207499) (end 186.432001 61.207499) (width 0.3) (layer B.Cu) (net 11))
 (segment (start 183.31 62.42) (end 184.522501 61.207499) (width 0.3) (layer B.Cu) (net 11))
 (segment (start 193.437501 63.282499) (end 194.3 62.42) (width 0.3) (layer B.Cu) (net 12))
 (segment (start 186.712499 63.282499) (end 193.437501 63.282499) (width 0.3) (layer B.Cu) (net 12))
 (segment (start 185.85 62.42) (end 186.712499 63.282499) (width 0.3) (layer B.Cu) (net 12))
 (segment (start 187.644502 59.88) (end 188.48 59.88) (width 0.3) (layer B.Cu) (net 9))
 (segment (start 184.637499 58.552501) (end 186.317003 58.552501) (width 0.3) (layer B.Cu) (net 9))
 (segment (start 186.317003 58.552501) (end 187.644502 59.88) (width 0.3) (layer B.Cu) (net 9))
 (segment (start 183.31 59.88) (end 184.637499 58.552501) (width 0.3) (layer B.Cu) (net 9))
 (segment (start 193.437501 60.742499) (end 194.3 59.88) (width 0.3) (layer B.Cu) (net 10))
 (segment (start 186.712499 60.742499) (end 193.437501 60.742499) (width 0.3) (layer B.Cu) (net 10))
 (segment (start 185.85 59.88) (end 186.712499 60.742499) (width 0.3) (layer B.Cu) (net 10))
 (segment (start 186.317003 56.012501) (end 187.644502 57.34) (width 0.3) (layer B.Cu) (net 7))
 (segment (start 184.017122 57.34) (end 185.344621 56.012501) (width 0.3) (layer B.Cu) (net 7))
 (segment (start 183.31 57.34) (end 184.017122 57.34) (width 0.3) (layer B.Cu) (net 7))
 (segment (start 185.344621 56.012501) (end 186.317003 56.012501) (width 0.3) (layer B.Cu) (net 7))
 (segment (start 187.644502 57.34) (end 188.48 57.34) (width 0.3) (layer B.Cu) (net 7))
 (segment (start 193.437501 58.202499) (end 194.3 57.34) (width 0.3) (layer B.Cu) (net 8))
 (segment (start 186.712499 58.202499) (end 193.437501 58.202499) (width 0.3) (layer B.Cu) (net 8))
 (segment (start 185.85 57.34) (end 186.712499 58.202499) (width 0.3) (layer B.Cu) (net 8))
 (segment (start 193.437501 55.662499) (end 194.3 54.8) (width 0.3) (layer B.Cu) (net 2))
 (segment (start 186.712499 55.662499) (end 193.437501 55.662499) (width 0.3) (layer B.Cu) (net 2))
 (segment (start 185.85 54.8) (end 186.712499 55.662499) (width 0.3) (layer B.Cu) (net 2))
 (segment (start 180.5412 42.4646) (end 187.0412 42.4646) (width 0.5) (layer F.Cu) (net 2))
 (segment (start 179.403699 43.602101) (end 180.5412 42.4646) (width 0.3) (layer B.Cu) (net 2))
 (segment (start 179.403699 47.493699) (end 179.403699 43.602101) (width 0.3) (layer B.Cu) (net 2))
 (segment (start 181.09 49.18) (end 179.403699 47.493699) (width 0.3) (layer B.Cu) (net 2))
 (segment (start 181.09 50.75) (end 181.09 49.18) (width 0.3) (layer B.Cu) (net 2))
 (segment (start 181.59 51.25) (end 181.09 50.75) (width 0.3) (layer B.Cu) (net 2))
 (segment (start 182.727999 56.012501) (end 181.59 54.874502) (width 0.3) (layer B.Cu) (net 2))
 (segment (start 184.637499 56.012501) (end 182.727999 56.012501) (width 0.3) (layer B.Cu) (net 2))
 (segment (start 181.59 54.874502) (end 181.59 51.25) (width 0.3) (layer B.Cu) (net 2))
 (segment (start 185.85 54.8) (end 184.637499 56.012501) (width 0.3) (layer B.Cu) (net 2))
 (segment (start 184.637499 50.932501) (end 187.152501 50.932501) (width 0.3) (layer B.Cu) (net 5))
 (segment (start 187.152501 50.932501) (end 188.48 52.26) (width 0.3) (layer B.Cu) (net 5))
 (segment (start 183.31 52.26) (end 184.637499 50.932501) (width 0.3) (layer B.Cu) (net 5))
 (segment (start 187.267499 48.507499) (end 188.48 49.72) (width 0.3) (layer B.Cu) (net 3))
 (segment (start 184.522501 48.507499) (end 187.267499 48.507499) (width 0.3) (layer B.Cu) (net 3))
 (segment (start 183.31 49.72) (end 184.522501 48.507499) (width 0.3) (layer B.Cu) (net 3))
 (segment (start 187.625002 54.8) (end 188.48 54.8) (width 0.3) (layer B.Cu) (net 1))
 (segment (start 186.412501 53.587499) (end 187.625002 54.8) (width 0.3) (layer B.Cu) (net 1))
 (segment (start 184.522501 53.587499) (end 186.412501 53.587499) (width 0.3) (layer B.Cu) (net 1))
 (segment (start 183.31 54.8) (end 184.522501 53.587499) (width 0.3) (layer B.Cu) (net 1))
 (segment (start 180.5412 46.9646) (end 187.0412 46.9646) (width 0.5) (layer F.Cu) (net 1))
 (segment (start 181.59749 50.46749) (end 181.59749 48.02089) (width 0.3) (layer B.Cu) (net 1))
 (segment (start 182.097499 50.967499) (end 181.59749 50.46749) (width 0.3) (layer B.Cu) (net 1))
 (segment (start 182.097499 53.587499) (end 182.097499 50.967499) (width 0.3) (layer B.Cu) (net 1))
 (segment (start 181.59749 48.02089) (end 180.5412 46.9646) (width 0.3) (layer B.Cu) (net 1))
 (segment (start 183.31 54.8) (end 182.097499 53.587499) (width 0.3) (layer B.Cu) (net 1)))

